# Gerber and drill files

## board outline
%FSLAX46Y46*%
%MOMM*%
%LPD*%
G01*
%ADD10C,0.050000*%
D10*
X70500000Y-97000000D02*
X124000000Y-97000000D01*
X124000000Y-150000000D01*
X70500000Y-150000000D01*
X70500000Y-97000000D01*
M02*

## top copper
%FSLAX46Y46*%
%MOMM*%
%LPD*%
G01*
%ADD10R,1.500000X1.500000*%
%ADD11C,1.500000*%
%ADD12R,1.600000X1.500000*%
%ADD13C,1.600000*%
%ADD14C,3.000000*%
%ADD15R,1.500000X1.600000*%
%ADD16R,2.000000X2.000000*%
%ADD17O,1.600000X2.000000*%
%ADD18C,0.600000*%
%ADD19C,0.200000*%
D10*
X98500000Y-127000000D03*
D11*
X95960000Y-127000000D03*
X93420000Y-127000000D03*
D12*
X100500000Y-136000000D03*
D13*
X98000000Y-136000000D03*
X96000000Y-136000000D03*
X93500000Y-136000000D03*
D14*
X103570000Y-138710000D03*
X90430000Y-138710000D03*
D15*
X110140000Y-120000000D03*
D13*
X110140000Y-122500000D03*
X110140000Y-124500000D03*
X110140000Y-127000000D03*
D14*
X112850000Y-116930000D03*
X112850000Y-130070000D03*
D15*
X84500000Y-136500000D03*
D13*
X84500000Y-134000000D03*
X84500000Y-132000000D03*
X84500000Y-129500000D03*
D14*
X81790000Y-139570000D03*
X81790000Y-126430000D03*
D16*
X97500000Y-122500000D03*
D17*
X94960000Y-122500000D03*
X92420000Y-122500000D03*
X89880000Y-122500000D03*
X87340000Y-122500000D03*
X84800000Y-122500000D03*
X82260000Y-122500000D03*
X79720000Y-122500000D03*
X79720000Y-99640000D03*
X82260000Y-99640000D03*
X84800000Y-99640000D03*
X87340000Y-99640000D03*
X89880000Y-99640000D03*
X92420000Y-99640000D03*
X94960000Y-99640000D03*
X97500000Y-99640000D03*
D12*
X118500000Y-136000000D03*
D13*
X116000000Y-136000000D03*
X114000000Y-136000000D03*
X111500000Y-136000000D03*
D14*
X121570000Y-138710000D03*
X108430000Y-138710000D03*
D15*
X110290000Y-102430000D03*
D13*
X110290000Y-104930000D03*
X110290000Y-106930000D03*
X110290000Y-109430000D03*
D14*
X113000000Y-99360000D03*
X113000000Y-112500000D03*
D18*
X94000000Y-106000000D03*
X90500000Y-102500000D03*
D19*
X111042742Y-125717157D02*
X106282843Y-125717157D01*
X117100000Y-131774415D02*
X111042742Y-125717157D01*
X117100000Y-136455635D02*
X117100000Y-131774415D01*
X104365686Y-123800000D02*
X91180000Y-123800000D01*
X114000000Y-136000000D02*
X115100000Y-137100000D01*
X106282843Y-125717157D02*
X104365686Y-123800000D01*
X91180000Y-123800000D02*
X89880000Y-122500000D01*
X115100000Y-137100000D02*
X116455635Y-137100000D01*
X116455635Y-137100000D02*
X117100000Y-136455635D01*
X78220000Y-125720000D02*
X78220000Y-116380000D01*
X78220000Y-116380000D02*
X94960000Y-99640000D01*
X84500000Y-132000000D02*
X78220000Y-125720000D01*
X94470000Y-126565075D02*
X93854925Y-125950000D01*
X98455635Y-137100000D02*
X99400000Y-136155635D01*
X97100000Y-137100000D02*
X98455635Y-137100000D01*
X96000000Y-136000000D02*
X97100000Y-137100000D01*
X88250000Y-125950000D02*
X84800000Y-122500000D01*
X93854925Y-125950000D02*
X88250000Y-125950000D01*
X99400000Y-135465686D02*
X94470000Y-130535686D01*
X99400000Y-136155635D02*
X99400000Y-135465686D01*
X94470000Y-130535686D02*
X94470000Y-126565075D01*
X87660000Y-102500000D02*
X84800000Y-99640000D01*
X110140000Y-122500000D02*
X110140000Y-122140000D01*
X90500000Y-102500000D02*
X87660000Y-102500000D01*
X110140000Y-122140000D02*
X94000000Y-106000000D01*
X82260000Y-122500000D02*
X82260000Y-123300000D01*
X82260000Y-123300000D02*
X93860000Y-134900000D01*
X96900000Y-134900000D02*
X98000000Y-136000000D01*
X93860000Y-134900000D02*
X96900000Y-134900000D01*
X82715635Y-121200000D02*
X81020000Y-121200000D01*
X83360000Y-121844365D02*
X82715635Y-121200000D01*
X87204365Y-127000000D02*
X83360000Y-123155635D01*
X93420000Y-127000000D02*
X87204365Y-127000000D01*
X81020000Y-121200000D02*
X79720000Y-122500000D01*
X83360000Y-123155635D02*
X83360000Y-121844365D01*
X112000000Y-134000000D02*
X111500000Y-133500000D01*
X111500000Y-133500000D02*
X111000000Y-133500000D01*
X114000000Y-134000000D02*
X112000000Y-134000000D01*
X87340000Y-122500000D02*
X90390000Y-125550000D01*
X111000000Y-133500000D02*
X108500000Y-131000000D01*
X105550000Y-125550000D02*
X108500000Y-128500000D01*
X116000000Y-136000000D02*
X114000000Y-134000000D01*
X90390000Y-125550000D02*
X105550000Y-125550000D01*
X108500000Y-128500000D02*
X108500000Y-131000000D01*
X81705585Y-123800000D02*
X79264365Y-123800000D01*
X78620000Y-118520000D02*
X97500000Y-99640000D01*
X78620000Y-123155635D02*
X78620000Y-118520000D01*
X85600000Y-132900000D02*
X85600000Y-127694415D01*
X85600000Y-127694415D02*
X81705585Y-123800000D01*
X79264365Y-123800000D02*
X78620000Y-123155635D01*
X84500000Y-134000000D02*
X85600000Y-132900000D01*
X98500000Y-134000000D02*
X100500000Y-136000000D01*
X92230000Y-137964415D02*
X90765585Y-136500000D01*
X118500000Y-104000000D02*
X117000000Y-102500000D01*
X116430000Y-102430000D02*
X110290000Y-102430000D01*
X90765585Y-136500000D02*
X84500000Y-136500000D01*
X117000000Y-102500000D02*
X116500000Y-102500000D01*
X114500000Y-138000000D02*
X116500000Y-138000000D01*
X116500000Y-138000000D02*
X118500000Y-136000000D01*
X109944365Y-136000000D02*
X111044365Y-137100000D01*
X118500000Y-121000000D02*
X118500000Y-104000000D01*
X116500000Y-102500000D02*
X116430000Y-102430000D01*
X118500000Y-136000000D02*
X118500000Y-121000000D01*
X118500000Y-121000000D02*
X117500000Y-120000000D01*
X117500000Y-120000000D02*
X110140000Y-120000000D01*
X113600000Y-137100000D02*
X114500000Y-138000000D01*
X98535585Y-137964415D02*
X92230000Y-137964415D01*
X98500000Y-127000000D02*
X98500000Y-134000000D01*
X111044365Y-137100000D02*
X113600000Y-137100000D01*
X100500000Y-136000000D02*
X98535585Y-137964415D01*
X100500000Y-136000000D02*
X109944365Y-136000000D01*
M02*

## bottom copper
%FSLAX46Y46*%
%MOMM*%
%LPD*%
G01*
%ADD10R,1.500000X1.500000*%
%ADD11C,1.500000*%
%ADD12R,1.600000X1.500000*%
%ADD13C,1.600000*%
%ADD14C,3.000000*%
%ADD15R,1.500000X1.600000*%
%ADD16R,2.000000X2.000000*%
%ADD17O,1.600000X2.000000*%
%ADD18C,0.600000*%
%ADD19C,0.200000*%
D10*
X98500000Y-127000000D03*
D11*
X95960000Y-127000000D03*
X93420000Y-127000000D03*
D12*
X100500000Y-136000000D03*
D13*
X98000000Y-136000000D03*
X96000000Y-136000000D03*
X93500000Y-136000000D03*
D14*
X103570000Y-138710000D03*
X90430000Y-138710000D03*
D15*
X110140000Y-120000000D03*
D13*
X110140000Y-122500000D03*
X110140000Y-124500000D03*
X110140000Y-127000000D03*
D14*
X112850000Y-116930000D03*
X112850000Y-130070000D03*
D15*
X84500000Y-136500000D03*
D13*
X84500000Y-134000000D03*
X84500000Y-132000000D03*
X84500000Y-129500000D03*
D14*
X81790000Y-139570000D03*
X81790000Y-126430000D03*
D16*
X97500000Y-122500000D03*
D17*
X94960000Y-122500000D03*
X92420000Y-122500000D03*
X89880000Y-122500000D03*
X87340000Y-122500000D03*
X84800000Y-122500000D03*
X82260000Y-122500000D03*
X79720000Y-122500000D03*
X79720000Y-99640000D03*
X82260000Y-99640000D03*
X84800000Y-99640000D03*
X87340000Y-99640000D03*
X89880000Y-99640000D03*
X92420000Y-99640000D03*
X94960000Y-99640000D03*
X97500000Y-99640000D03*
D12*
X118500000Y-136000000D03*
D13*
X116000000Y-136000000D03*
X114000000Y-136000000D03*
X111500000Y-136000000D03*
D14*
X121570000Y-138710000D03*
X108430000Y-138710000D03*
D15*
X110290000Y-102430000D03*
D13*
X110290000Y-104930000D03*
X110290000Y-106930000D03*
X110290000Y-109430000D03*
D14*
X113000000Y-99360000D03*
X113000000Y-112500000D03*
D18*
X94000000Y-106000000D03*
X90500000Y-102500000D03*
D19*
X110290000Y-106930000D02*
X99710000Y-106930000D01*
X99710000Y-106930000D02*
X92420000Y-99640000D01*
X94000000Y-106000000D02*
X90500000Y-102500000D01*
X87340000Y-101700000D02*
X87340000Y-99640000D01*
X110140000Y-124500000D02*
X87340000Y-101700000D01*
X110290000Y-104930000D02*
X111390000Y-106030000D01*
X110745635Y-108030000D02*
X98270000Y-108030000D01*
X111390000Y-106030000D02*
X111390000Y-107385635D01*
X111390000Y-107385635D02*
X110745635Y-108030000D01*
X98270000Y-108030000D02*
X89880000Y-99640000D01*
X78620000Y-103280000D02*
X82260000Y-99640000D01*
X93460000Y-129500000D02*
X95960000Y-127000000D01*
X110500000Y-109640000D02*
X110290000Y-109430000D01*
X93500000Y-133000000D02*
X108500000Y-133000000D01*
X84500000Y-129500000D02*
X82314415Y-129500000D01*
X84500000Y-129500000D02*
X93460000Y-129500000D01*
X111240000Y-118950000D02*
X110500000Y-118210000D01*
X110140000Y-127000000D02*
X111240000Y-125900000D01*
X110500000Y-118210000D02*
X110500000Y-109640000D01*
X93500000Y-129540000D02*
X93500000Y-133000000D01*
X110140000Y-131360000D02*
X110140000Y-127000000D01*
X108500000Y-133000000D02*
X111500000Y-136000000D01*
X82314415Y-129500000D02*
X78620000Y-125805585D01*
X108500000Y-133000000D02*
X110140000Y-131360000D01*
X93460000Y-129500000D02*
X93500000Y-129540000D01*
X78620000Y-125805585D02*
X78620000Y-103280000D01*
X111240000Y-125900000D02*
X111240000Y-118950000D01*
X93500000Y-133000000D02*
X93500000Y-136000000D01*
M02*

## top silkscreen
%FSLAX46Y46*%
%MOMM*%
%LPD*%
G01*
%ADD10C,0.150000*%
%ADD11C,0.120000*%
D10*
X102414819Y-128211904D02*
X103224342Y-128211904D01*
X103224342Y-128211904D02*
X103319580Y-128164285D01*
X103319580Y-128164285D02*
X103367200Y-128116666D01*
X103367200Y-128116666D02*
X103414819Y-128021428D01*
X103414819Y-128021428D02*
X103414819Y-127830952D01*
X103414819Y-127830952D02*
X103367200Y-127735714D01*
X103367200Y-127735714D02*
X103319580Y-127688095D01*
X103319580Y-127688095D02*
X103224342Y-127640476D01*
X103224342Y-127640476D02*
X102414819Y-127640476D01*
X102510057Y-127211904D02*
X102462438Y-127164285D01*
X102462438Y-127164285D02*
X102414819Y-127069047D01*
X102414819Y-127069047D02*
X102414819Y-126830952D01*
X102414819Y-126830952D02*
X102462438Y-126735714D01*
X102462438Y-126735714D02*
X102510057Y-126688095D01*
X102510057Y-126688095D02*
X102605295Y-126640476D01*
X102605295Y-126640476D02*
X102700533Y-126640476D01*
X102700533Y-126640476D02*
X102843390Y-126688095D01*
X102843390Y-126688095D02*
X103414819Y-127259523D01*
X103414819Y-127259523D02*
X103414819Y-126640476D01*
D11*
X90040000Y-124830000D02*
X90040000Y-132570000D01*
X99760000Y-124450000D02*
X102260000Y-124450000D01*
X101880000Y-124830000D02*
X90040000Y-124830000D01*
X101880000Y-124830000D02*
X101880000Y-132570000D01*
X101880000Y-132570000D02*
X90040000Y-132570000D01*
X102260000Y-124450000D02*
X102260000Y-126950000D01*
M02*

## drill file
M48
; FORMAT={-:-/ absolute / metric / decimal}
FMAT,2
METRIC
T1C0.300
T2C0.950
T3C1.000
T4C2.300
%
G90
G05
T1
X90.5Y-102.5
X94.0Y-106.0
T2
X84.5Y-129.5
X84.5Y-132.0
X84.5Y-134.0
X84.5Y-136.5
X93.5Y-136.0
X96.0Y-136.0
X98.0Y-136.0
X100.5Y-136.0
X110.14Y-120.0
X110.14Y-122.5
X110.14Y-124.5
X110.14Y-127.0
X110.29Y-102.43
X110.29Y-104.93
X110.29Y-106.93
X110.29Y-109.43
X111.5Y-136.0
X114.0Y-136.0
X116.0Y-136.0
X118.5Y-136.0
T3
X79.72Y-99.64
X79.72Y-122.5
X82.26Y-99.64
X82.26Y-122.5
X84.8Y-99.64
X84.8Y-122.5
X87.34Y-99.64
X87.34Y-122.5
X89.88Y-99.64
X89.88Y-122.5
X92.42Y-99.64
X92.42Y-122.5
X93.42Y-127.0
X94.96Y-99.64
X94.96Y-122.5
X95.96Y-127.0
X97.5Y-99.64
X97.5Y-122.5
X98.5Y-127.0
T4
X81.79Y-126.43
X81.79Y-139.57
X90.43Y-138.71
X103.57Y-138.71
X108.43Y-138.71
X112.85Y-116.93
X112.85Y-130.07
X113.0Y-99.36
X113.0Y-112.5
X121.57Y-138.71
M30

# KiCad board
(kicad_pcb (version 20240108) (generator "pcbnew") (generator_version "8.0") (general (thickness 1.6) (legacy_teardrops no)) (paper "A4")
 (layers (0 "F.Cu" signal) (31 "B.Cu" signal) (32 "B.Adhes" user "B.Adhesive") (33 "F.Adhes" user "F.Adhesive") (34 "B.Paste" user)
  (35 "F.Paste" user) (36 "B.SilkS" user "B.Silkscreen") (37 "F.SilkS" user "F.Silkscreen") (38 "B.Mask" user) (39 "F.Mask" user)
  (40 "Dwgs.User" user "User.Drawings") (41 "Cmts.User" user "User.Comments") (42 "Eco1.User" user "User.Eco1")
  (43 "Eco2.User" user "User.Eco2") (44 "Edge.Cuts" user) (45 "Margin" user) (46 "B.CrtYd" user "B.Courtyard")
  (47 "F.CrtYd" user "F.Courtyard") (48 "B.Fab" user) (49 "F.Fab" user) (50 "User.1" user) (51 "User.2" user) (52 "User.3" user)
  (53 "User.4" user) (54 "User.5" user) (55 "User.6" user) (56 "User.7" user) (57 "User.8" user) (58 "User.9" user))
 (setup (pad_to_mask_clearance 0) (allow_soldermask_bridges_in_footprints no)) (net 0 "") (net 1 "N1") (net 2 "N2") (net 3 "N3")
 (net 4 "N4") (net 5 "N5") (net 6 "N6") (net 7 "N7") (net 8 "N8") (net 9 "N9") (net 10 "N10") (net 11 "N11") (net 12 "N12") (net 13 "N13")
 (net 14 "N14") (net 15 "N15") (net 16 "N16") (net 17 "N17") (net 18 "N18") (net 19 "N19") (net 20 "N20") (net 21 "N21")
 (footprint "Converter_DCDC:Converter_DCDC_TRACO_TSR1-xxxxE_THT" (layer "F.Cu") (at 98.5 127 -90)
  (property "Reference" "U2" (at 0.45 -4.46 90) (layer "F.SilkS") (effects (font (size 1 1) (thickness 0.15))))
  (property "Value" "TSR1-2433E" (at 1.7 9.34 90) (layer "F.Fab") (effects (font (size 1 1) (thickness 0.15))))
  (fp_line (start -2.17 8.46) (end 5.57 8.46) (stroke (width 0.12) (type solid)) (layer "F.SilkS"))
  (fp_line (start -2.55 -1.26) (end -2.55 -3.76) (stroke (width 0.12) (type solid)) (layer "F.SilkS"))
  (fp_line (start -2.17 -3.38) (end -2.17 8.46) (stroke (width 0.12) (type solid)) (layer "F.SilkS"))
  (fp_line (start -2.17 -3.38) (end 5.57 -3.38) (stroke (width 0.12) (type solid)) (layer "F.SilkS"))
  (fp_line (start 5.57 -3.38) (end 5.57 8.46) (stroke (width 0.12) (type solid)) (layer "F.SilkS"))
  (fp_line (start -2.55 -3.76) (end -0.05 -3.76) (stroke (width 0.12) (type solid)) (layer "F.SilkS"))
  (pad "1" thru_hole rect (at 0 0 270) (size 1.5 1.5) (drill 1) (layers "*.Cu" "*.Mask") (remove_unused_layers no) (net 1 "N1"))
  (pad "2" thru_hole circle (at 0 2.54 270) (size 1.5 1.5) (drill 1) (layers "*.Cu" "*.Mask") (remove_unused_layers no) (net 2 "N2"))
  (pad "3" thru_hole circle (at 0 5.08 270) (size 1.5 1.5) (drill 1) (layers "*.Cu" "*.Mask") (remove_unused_layers no) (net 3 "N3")))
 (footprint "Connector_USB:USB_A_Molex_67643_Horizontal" (layer "B.Cu") (at 100.5 136 180)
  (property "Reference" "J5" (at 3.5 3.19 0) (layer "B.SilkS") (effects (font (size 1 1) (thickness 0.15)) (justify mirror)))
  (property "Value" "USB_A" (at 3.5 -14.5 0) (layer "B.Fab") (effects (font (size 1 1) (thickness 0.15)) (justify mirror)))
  (pad "1" thru_hole rect (at 0 0 180) (size 1.6 1.5) (drill 0.95) (layers "*.Cu" "*.Mask") (remove_unused_layers no) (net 1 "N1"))
  (pad "2" thru_hole circle (at 2.5 0 180) (size 1.6 1.6) (drill 0.95) (layers "*.Cu" "*.Mask") (remove_unused_layers no) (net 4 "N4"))
  (pad "3" thru_hole circle (at 4.5 0 180) (size 1.6 1.6) (drill 0.95) (layers "*.Cu" "*.Mask") (remove_unused_layers no) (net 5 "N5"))
  (pad "4" thru_hole circle (at 7 0 180) (size 1.6 1.6) (drill 0.95) (layers "*.Cu" "*.Mask") (remove_unused_layers no) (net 2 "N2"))
  (pad "5" thru_hole circle (at -3.07 -2.71 180) (size 3 3) (drill 2.3) (layers "*.Cu" "*.Mask") (remove_unused_layers no) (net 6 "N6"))
  (pad "5" thru_hole circle (at 10.07 -2.71 180) (size 3 3) (drill 2.3) (layers "*.Cu" "*.Mask") (remove_unused_layers no) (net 6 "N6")))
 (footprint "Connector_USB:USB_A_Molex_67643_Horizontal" (layer "B.Cu") (at 110.14 120 -90)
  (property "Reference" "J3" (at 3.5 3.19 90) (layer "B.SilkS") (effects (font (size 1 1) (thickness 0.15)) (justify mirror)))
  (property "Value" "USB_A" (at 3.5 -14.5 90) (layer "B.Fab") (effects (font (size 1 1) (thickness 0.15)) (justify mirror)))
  (pad "1" thru_hole rect (at 0 0 270) (size 1.6 1.5) (drill 0.95) (layers "*.Cu" "*.Mask") (remove_unused_layers no) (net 1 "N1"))
  (pad "2" thru_hole circle (at 2.5 0 270) (size 1.6 1.6) (drill 0.95) (layers "*.Cu" "*.Mask") (remove_unused_layers no) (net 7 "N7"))
  (pad "3" thru_hole circle (at 4.5 0 270) (size 1.6 1.6) (drill 0.95) (layers "*.Cu" "*.Mask") (remove_unused_layers no) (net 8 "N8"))
  (pad "4" thru_hole circle (at 7 0 270) (size 1.6 1.6) (drill 0.95) (layers "*.Cu" "*.Mask") (remove_unused_layers no) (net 2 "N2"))
  (pad "5" thru_hole circle (at -3.07 -2.71 270) (size 3 3) (drill 2.3) (layers "*.Cu" "*.Mask") (remove_unused_layers no) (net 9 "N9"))
  (pad "5" thru_hole circle (at 10.07 -2.71 270) (size 3 3) (drill 2.3) (layers "*.Cu" "*.Mask") (remove_unused_layers no) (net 9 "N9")))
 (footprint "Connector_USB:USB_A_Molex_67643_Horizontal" (layer "B.Cu") (at 84.5 136.5 90)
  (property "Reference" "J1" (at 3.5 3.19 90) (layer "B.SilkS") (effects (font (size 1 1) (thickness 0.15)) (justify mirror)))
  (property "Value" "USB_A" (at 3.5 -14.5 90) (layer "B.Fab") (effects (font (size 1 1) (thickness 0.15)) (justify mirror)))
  (pad "1" thru_hole rect (at 0 0 90) (size 1.6 1.5) (drill 0.95) (layers "*.Cu" "*.Mask") (remove_unused_layers no) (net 1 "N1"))
  (pad "2" thru_hole circle (at 2.5 0 90) (size 1.6 1.6) (drill 0.95) (layers "*.Cu" "*.Mask") (remove_unused_layers no) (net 2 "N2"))
  (pad "3" thru_hole circle (at 4.5 0 90) (size 1.6 1.6) (drill 0.95) (layers "*.Cu" "*.Mask") (remove_unused_layers no) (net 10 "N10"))
  (pad "4" thru_hole circle (at 7 0 90) (size 1.6 1.6) (drill 0.95) (layers "*.Cu" "*.Mask") (remove_unused_layers no) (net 2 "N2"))
  (pad "5" thru_hole circle (at -3.07 -2.71 90) (size 3 3) (drill 2.3) (layers "*.Cu" "*.Mask") (remove_unused_layers no) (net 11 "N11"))
  (pad "5" thru_hole circle (at 10.07 -2.71 90) (size 3 3) (drill 2.3) (layers "*.Cu" "*.Mask") (remove_unused_layers no) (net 11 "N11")))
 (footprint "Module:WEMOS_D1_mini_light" (layer "B.Cu") (at 97.5 122.5 90)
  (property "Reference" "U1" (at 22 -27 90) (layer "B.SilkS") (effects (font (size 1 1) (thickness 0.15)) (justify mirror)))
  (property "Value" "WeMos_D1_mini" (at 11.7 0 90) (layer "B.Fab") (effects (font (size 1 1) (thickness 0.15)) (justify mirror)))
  (pad "1" thru_hole rect (at 0 0 90) (size 2 2) (drill 1) (layers "*.Cu" "*.Mask") (remove_unused_layers no) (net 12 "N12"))
  (pad "2" thru_hole oval (at 0 -2.54 90) (size 2 1.6) (drill 1) (layers "*.Cu" "*.Mask") (remove_unused_layers no) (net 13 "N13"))
  (pad "3" thru_hole oval (at 0 -5.08 90) (size 2 1.6) (drill 1) (layers "*.Cu" "*.Mask") (remove_unused_layers no) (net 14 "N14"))
  (pad "4" thru_hole oval (at 0 -7.62 90) (size 2 1.6) (drill 1) (layers "*.Cu" "*.Mask") (remove_unused_layers no) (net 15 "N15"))
  (pad "5" thru_hole oval (at 0 -10.16 90) (size 2 1.6) (drill 1) (layers "*.Cu" "*.Mask") (remove_unused_layers no) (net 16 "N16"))
  (pad "6" thru_hole oval (at 0 -12.7 90) (size 2 1.6) (drill 1) (layers "*.Cu" "*.Mask") (remove_unused_layers no) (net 5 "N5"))
  (pad "7" thru_hole oval (at 0 -15.24 90) (size 2 1.6) (drill 1) (layers "*.Cu" "*.Mask") (remove_unused_layers no) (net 4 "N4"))
  (pad "8" thru_hole oval (at 0 -17.78 90) (size 2 1.6) (drill 1) (layers "*.Cu" "*.Mask") (remove_unused_layers no) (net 3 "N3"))
  (pad "9" thru_hole oval (at 22.86 -17.78 90) (size 2 1.6) (drill 1) (layers "*.Cu" "*.Mask") (remove_unused_layers no) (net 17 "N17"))
  (pad "10" thru_hole oval (at 22.86 -15.24 90) (size 2 1.6) (drill 1) (layers "*.Cu" "*.Mask") (remove_unused_layers no) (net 2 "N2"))
  (pad "11" thru_hole oval (at 22.86 -12.7 90) (size 2 1.6) (drill 1) (layers "*.Cu" "*.Mask") (remove_unused_layers no) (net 7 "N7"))
  (pad "12" thru_hole oval (at 22.86 -10.16 90) (size 2 1.6) (drill 1) (layers "*.Cu" "*.Mask") (remove_unused_layers no) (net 8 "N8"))
  (pad "13" thru_hole oval (at 22.86 -7.62 90) (size 2 1.6) (drill 1) (layers "*.Cu" "*.Mask") (remove_unused_layers no) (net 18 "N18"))
  (pad "14" thru_hole oval (at 22.86 -5.08 90) (size 2 1.6) (drill 1) (layers "*.Cu" "*.Mask") (remove_unused_layers no) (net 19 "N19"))
  (pad "15" thru_hole oval (at 22.86 -2.54 90) (size 2 1.6) (drill 1) (layers "*.Cu" "*.Mask") (remove_unused_layers no) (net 10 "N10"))
  (pad "16" thru_hole oval (at 22.86 0 90) (size 2 1.6) (drill 1) (layers "*.Cu" "*.Mask") (remove_unused_layers no) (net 2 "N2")))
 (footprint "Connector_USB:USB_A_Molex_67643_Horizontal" (layer "B.Cu") (at 118.5 136 180)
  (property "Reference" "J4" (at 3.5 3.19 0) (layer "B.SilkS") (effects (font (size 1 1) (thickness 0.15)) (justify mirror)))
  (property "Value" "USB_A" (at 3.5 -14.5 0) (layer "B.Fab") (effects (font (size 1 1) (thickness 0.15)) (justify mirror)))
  (pad "1" thru_hole rect (at 0 0 180) (size 1.6 1.5) (drill 0.95) (layers "*.Cu" "*.Mask") (remove_unused_layers no) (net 1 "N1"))
  (pad "2" thru_hole circle (at 2.5 0 180) (size 1.6 1.6) (drill 0.95) (layers "*.Cu" "*.Mask") (remove_unused_layers no) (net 16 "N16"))
  (pad "3" thru_hole circle (at 4.5 0 180) (size 1.6 1.6) (drill 0.95) (layers "*.Cu" "*.Mask") (remove_unused_layers no) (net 15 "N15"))
  (pad "4" thru_hole circle (at 7 0 180) (size 1.6 1.6) (drill 0.95) (layers "*.Cu" "*.Mask") (remove_unused_layers no) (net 2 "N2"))
  (pad "5" thru_hole circle (at -3.07 -2.71 180) (size 3 3) (drill 2.3) (layers "*.Cu" "*.Mask") (remove_unused_layers no) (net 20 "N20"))
  (pad "5" thru_hole circle (at 10.07 -2.71 180) (size 3 3) (drill 2.3) (layers "*.Cu" "*.Mask") (remove_unused_layers no) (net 20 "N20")))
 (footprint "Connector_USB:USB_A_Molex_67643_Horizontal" (layer "B.Cu") (at 110.29 102.43 -90)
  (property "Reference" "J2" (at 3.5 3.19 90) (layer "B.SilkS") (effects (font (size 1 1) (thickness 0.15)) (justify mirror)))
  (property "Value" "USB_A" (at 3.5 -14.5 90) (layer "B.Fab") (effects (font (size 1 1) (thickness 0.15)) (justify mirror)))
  (pad "1" thru_hole rect (at 0 0 270) (size 1.6 1.5) (drill 0.95) (layers "*.Cu" "*.Mask") (remove_unused_layers no) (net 1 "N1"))
  (pad "2" thru_hole circle (at 2.5 0 270) (size 1.6 1.6) (drill 0.95) (layers "*.Cu" "*.Mask") (remove_unused_layers no) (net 18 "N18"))
  (pad "3" thru_hole circle (at 4.5 0 270) (size 1.6 1.6) (drill 0.95) (layers "*.Cu" "*.Mask") (remove_unused_layers no) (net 19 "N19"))
  (pad "4" thru_hole circle (at 7 0 270) (size 1.6 1.6) (drill 0.95) (layers "*.Cu" "*.Mask") (remove_unused_layers no) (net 2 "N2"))
  (pad "5" thru_hole circle (at -3.07 -2.71 270) (size 3 3) (drill 2.3) (layers "*.Cu" "*.Mask") (remove_unused_layers no) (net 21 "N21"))
  (pad "5" thru_hole circle (at 10.07 -2.71 270) (size 3 3) (drill 2.3) (layers "*.Cu" "*.Mask") (remove_unused_layers no) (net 21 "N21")))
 (gr_rect (start 70.5 97) (end 124 150) (stroke (width 0.05) (type default)) (fill none) (layer "Edge.Cuts"))
 (segment (start 110.29 106.93) (end 99.71 106.93) (width 0.2) (layer "B.Cu") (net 19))
 (segment (start 99.71 106.93) (end 92.42 99.64) (width 0.2) (layer "B.Cu") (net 19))
 (segment (start 111.042742 125.717157) (end 106.282843 125.717157) (width 0.2) (layer "F.Cu") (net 15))
 (segment (start 117.1 131.774415) (end 111.042742 125.717157) (width 0.2) (layer "F.Cu") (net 15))
 (segment (start 117.1 136.455635) (end 117.1 131.774415) (width 0.2) (layer "F.Cu") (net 15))
 (segment (start 104.365686 123.8) (end 91.18 123.8) (width 0.2) (layer "F.Cu") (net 15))
 (segment (start 114 136) (end 115.1 137.1) (width 0.2) (layer "F.Cu") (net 15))
 (segment (start 106.282843 125.717157) (end 104.365686 123.8) (width 0.2) (layer "F.Cu") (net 15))
 (segment (start 91.18 123.8) (end 89.88 122.5) (width 0.2) (layer "F.Cu") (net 15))
 (segment (start 115.1 137.1) (end 116.455635 137.1) (width 0.2) (layer "F.Cu") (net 15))
 (segment (start 116.455635 137.1) (end 117.1 136.455635) (width 0.2) (layer "F.Cu") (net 15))
 (segment (start 78.22 125.72) (end 78.22 116.38) (width 0.2) (layer "F.Cu") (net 10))
 (segment (start 78.22 116.38) (end 94.96 99.64) (width 0.2) (layer "F.Cu") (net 10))
 (segment (start 84.5 132) (end 78.22 125.72) (width 0.2) (layer "F.Cu") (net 10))
 (segment (start 94.47 126.565075) (end 93.854925 125.95) (width 0.2) (layer "F.Cu") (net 5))
 (segment (start 98.455635 137.1) (end 99.4 136.155635) (width 0.2) (layer "F.Cu") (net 5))
 (segment (start 97.1 137.1) (end 98.455635 137.1) (width 0.2) (layer "F.Cu") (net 5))
 (segment (start 96 136) (end 97.1 137.1) (width 0.2) (layer "F.Cu") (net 5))
 (segment (start 88.25 125.95) (end 84.8 122.5) (width 0.2) (layer "F.Cu") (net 5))
 (segment (start 93.854925 125.95) (end 88.25 125.95) (width 0.2) (layer "F.Cu") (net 5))
 (segment (start 99.4 135.465686) (end 94.47 130.535686) (width 0.2) (layer "F.Cu") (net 5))
 (segment (start 99.4 136.155635) (end 99.4 135.465686) (width 0.2) (layer "F.Cu") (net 5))
 (segment (start 94.47 130.535686) (end 94.47 126.565075) (width 0.2) (layer "F.Cu") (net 5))
 (segment (start 87.66 102.5) (end 84.8 99.64) (width 0.2) (layer "F.Cu") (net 7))
 (segment (start 110.14 122.5) (end 110.14 122.14) (width 0.2) (layer "F.Cu") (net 7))
 (segment (start 90.5 102.5) (end 87.66 102.5) (width 0.2) (layer "F.Cu") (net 7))
 (segment (start 110.14 122.14) (end 94 106) (width 0.2) (layer "F.Cu") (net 7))
 (via (at 94 106) (size 0.6) (drill 0.3) (layers "F.Cu" "B.Cu") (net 7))
 (via (at 90.5 102.5) (size 0.6) (drill 0.3) (layers "F.Cu" "B.Cu") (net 7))
 (segment (start 94 106) (end 90.5 102.5) (width 0.2) (layer "B.Cu") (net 7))
 (segment (start 82.26 122.5) (end 82.26 123.3) (width 0.2) (layer "F.Cu") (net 4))
 (segment (start 82.26 123.3) (end 93.86 134.9) (width 0.2) (layer "F.Cu") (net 4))
 (segment (start 96.9 134.9) (end 98 136) (width 0.2) (layer "F.Cu") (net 4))
 (segment (start 93.86 134.9) (end 96.9 134.9) (width 0.2) (layer "F.Cu") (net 4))
 (segment (start 87.34 101.7) (end 87.34 99.64) (width 0.2) (layer "B.Cu") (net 8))
 (segment (start 110.14 124.5) (end 87.34 101.7) (width 0.2) (layer "B.Cu") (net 8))
 (segment (start 110.29 104.93) (end 111.39 106.03) (width 0.2) (layer "B.Cu") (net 18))
 (segment (start 110.745635 108.03) (end 98.27 108.03) (width 0.2) (layer "B.Cu") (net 18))
 (segment (start 111.39 106.03) (end 111.39 107.385635) (width 0.2) (layer "B.Cu") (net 18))
 (segment (start 111.39 107.385635) (end 110.745635 108.03) (width 0.2) (layer "B.Cu") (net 18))
 (segment (start 98.27 108.03) (end 89.88 99.64) (width 0.2) (layer "B.Cu") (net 18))
 (segment (start 82.715635 121.2) (end 81.02 121.2) (width 0.2) (layer "F.Cu") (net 3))
 (segment (start 83.36 121.844365) (end 82.715635 121.2) (width 0.2) (layer "F.Cu") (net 3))
 (segment (start 87.204365 127) (end 83.36 123.155635) (width 0.2) (layer "F.Cu") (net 3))
 (segment (start 93.42 127) (end 87.204365 127) (width 0.2) (layer "F.Cu") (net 3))
 (segment (start 81.02 121.2) (end 79.72 122.5) (width 0.2) (layer "F.Cu") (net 3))
 (segment (start 83.36 123.155635) (end 83.36 121.844365) (width 0.2) (layer "F.Cu") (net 3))
 (segment (start 112 134) (end 111.5 133.5) (width 0.2) (layer "F.Cu") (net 16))
 (segment (start 111.5 133.5) (end 111 133.5) (width 0.2) (layer "F.Cu") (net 16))
 (segment (start 114 134) (end 112 134) (width 0.2) (layer "F.Cu") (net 16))
 (segment (start 87.34 122.5) (end 90.39 125.55) (width 0.2) (layer "F.Cu") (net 16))
 (segment (start 111 133.5) (end 108.5 131) (width 0.2) (layer "F.Cu") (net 16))
 (segment (start 105.55 125.55) (end 108.5 128.5) (width 0.2) (layer "F.Cu") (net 16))
 (segment (start 116 136) (end 114 134) (width 0.2) (layer "F.Cu") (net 16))
 (segment (start 90.39 125.55) (end 105.55 125.55) (width 0.2) (layer "F.Cu") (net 16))
 (segment (start 108.5 128.5) (end 108.5 131) (width 0.2) (layer "F.Cu") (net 16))
 (segment (start 81.705585 123.8) (end 79.264365 123.8) (width 0.2) (layer "F.Cu") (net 2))
 (segment (start 78.62 118.52) (end 97.5 99.64) (width 0.2) (layer "F.Cu") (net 2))
 (segment (start 78.62 123.155635) (end 78.62 118.52) (width 0.2) (layer "F.Cu") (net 2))
 (segment (start 85.6 132.9) (end 85.6 127.694415) (width 0.2) (layer "F.Cu") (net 2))
 (segment (start 85.6 127.694415) (end 81.705585 123.8) (width 0.2) (layer "F.Cu") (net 2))
 (segment (start 79.264365 123.8) (end 78.62 123.155635) (width 0.2) (layer "F.Cu") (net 2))
 (segment (start 84.5 134) (end 85.6 132.9) (width 0.2) (layer "F.Cu") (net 2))
 (segment (start 78.62 103.28) (end 82.26 99.64) (width 0.2) (layer "B.Cu") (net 2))
 (segment (start 93.46 129.5) (end 95.96 127) (width 0.2) (layer "B.Cu") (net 2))
 (segment (start 110.5 109.64) (end 110.29 109.43) (width 0.2) (layer "B.Cu") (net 2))
 (segment (start 93.5 133) (end 108.5 133) (width 0.2) (layer "B.Cu") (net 2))
 (segment (start 84.5 129.5) (end 82.314415 129.5) (width 0.2) (layer "B.Cu") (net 2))
 (segment (start 84.5 129.5) (end 93.46 129.5) (width 0.2) (layer "B.Cu") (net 2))
 (segment (start 111.24 118.95) (end 110.5 118.21) (width 0.2) (layer "B.Cu") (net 2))
 (segment (start 110.14 127) (end 111.24 125.9) (width 0.2) (layer "B.Cu") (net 2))
 (segment (start 110.5 118.21) (end 110.5 109.64) (width 0.2) (layer "B.Cu") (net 2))
 (segment (start 93.5 129.54) (end 93.5 133) (width 0.2) (layer "B.Cu") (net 2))
 (segment (start 110.14 131.36) (end 110.14 127) (width 0.2) (layer "B.Cu") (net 2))
 (segment (start 108.5 133) (end 111.5 136) (width 0.2) (layer "B.Cu") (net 2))
 (segment (start 82.314415 129.5) (end 78.62 125.805585) (width 0.2) (layer "B.Cu") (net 2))
 (segment (start 108.5 133) (end 110.14 131.36) (width 0.2) (layer "B.Cu") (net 2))
 (segment (start 93.46 129.5) (end 93.5 129.54) (width 0.2) (layer "B.Cu") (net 2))
 (segment (start 78.62 125.805585) (end 78.62 103.28) (width 0.2) (layer "B.Cu") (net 2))
 (segment (start 111.24 125.9) (end 111.24 118.95) (width 0.2) (layer "B.Cu") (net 2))
 (segment (start 93.5 133) (end 93.5 136) (width 0.2) (layer "B.Cu") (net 2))
 (segment (start 98.5 134) (end 100.5 136) (width 0.2) (layer "F.Cu") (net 1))
 (segment (start 92.23 137.964415) (end 90.765585 136.5) (width 0.2) (layer "F.Cu") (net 1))
 (segment (start 118.5 104) (end 117 102.5) (width 0.2) (layer "F.Cu") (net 1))
 (segment (start 116.43 102.43) (end 110.29 102.43) (width 0.2) (layer "F.Cu") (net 1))
 (segment (start 90.765585 136.5) (end 84.5 136.5) (width 0.2) (layer "F.Cu") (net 1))
 (segment (start 117 102.5) (end 116.5 102.5) (width 0.2) (layer "F.Cu") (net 1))
 (segment (start 114.5 138) (end 116.5 138) (width 0.2) (layer "F.Cu") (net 1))
 (segment (start 116.5 138) (end 118.5 136) (width 0.2) (layer "F.Cu") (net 1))
 (segment (start 109.944365 136) (end 111.044365 137.1) (width 0.2) (layer "F.Cu") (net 1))
 (segment (start 118.5 121) (end 118.5 104) (width 0.2) (layer "F.Cu") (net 1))
 (segment (start 116.5 102.5) (end 116.43 102.43) (width 0.2) (layer "F.Cu") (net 1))
 (segment (start 118.5 136) (end 118.5 121) (width 0.2) (layer "F.Cu") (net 1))
 (segment (start 118.5 121) (end 117.5 120) (width 0.2) (layer "F.Cu") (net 1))
 (segment (start 117.5 120) (end 110.14 120) (width 0.2) (layer "F.Cu") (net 1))
 (segment (start 113.6 137.1) (end 114.5 138) (width 0.2) (layer "F.Cu") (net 1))
 (segment (start 98.535585 137.964415) (end 92.23 137.964415) (width 0.2) (layer "F.Cu") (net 1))
 (segment (start 98.5 127) (end 98.5 134) (width 0.2) (layer "F.Cu") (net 1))
 (segment (start 111.044365 137.1) (end 113.6 137.1) (width 0.2) (layer "F.Cu") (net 1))
 (segment (start 100.5 136) (end 98.535585 137.964415) (width 0.2) (layer "F.Cu") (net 1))
 (segment (start 100.5 136) (end 109.944365 136) (width 0.2) (layer "F.Cu") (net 1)))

